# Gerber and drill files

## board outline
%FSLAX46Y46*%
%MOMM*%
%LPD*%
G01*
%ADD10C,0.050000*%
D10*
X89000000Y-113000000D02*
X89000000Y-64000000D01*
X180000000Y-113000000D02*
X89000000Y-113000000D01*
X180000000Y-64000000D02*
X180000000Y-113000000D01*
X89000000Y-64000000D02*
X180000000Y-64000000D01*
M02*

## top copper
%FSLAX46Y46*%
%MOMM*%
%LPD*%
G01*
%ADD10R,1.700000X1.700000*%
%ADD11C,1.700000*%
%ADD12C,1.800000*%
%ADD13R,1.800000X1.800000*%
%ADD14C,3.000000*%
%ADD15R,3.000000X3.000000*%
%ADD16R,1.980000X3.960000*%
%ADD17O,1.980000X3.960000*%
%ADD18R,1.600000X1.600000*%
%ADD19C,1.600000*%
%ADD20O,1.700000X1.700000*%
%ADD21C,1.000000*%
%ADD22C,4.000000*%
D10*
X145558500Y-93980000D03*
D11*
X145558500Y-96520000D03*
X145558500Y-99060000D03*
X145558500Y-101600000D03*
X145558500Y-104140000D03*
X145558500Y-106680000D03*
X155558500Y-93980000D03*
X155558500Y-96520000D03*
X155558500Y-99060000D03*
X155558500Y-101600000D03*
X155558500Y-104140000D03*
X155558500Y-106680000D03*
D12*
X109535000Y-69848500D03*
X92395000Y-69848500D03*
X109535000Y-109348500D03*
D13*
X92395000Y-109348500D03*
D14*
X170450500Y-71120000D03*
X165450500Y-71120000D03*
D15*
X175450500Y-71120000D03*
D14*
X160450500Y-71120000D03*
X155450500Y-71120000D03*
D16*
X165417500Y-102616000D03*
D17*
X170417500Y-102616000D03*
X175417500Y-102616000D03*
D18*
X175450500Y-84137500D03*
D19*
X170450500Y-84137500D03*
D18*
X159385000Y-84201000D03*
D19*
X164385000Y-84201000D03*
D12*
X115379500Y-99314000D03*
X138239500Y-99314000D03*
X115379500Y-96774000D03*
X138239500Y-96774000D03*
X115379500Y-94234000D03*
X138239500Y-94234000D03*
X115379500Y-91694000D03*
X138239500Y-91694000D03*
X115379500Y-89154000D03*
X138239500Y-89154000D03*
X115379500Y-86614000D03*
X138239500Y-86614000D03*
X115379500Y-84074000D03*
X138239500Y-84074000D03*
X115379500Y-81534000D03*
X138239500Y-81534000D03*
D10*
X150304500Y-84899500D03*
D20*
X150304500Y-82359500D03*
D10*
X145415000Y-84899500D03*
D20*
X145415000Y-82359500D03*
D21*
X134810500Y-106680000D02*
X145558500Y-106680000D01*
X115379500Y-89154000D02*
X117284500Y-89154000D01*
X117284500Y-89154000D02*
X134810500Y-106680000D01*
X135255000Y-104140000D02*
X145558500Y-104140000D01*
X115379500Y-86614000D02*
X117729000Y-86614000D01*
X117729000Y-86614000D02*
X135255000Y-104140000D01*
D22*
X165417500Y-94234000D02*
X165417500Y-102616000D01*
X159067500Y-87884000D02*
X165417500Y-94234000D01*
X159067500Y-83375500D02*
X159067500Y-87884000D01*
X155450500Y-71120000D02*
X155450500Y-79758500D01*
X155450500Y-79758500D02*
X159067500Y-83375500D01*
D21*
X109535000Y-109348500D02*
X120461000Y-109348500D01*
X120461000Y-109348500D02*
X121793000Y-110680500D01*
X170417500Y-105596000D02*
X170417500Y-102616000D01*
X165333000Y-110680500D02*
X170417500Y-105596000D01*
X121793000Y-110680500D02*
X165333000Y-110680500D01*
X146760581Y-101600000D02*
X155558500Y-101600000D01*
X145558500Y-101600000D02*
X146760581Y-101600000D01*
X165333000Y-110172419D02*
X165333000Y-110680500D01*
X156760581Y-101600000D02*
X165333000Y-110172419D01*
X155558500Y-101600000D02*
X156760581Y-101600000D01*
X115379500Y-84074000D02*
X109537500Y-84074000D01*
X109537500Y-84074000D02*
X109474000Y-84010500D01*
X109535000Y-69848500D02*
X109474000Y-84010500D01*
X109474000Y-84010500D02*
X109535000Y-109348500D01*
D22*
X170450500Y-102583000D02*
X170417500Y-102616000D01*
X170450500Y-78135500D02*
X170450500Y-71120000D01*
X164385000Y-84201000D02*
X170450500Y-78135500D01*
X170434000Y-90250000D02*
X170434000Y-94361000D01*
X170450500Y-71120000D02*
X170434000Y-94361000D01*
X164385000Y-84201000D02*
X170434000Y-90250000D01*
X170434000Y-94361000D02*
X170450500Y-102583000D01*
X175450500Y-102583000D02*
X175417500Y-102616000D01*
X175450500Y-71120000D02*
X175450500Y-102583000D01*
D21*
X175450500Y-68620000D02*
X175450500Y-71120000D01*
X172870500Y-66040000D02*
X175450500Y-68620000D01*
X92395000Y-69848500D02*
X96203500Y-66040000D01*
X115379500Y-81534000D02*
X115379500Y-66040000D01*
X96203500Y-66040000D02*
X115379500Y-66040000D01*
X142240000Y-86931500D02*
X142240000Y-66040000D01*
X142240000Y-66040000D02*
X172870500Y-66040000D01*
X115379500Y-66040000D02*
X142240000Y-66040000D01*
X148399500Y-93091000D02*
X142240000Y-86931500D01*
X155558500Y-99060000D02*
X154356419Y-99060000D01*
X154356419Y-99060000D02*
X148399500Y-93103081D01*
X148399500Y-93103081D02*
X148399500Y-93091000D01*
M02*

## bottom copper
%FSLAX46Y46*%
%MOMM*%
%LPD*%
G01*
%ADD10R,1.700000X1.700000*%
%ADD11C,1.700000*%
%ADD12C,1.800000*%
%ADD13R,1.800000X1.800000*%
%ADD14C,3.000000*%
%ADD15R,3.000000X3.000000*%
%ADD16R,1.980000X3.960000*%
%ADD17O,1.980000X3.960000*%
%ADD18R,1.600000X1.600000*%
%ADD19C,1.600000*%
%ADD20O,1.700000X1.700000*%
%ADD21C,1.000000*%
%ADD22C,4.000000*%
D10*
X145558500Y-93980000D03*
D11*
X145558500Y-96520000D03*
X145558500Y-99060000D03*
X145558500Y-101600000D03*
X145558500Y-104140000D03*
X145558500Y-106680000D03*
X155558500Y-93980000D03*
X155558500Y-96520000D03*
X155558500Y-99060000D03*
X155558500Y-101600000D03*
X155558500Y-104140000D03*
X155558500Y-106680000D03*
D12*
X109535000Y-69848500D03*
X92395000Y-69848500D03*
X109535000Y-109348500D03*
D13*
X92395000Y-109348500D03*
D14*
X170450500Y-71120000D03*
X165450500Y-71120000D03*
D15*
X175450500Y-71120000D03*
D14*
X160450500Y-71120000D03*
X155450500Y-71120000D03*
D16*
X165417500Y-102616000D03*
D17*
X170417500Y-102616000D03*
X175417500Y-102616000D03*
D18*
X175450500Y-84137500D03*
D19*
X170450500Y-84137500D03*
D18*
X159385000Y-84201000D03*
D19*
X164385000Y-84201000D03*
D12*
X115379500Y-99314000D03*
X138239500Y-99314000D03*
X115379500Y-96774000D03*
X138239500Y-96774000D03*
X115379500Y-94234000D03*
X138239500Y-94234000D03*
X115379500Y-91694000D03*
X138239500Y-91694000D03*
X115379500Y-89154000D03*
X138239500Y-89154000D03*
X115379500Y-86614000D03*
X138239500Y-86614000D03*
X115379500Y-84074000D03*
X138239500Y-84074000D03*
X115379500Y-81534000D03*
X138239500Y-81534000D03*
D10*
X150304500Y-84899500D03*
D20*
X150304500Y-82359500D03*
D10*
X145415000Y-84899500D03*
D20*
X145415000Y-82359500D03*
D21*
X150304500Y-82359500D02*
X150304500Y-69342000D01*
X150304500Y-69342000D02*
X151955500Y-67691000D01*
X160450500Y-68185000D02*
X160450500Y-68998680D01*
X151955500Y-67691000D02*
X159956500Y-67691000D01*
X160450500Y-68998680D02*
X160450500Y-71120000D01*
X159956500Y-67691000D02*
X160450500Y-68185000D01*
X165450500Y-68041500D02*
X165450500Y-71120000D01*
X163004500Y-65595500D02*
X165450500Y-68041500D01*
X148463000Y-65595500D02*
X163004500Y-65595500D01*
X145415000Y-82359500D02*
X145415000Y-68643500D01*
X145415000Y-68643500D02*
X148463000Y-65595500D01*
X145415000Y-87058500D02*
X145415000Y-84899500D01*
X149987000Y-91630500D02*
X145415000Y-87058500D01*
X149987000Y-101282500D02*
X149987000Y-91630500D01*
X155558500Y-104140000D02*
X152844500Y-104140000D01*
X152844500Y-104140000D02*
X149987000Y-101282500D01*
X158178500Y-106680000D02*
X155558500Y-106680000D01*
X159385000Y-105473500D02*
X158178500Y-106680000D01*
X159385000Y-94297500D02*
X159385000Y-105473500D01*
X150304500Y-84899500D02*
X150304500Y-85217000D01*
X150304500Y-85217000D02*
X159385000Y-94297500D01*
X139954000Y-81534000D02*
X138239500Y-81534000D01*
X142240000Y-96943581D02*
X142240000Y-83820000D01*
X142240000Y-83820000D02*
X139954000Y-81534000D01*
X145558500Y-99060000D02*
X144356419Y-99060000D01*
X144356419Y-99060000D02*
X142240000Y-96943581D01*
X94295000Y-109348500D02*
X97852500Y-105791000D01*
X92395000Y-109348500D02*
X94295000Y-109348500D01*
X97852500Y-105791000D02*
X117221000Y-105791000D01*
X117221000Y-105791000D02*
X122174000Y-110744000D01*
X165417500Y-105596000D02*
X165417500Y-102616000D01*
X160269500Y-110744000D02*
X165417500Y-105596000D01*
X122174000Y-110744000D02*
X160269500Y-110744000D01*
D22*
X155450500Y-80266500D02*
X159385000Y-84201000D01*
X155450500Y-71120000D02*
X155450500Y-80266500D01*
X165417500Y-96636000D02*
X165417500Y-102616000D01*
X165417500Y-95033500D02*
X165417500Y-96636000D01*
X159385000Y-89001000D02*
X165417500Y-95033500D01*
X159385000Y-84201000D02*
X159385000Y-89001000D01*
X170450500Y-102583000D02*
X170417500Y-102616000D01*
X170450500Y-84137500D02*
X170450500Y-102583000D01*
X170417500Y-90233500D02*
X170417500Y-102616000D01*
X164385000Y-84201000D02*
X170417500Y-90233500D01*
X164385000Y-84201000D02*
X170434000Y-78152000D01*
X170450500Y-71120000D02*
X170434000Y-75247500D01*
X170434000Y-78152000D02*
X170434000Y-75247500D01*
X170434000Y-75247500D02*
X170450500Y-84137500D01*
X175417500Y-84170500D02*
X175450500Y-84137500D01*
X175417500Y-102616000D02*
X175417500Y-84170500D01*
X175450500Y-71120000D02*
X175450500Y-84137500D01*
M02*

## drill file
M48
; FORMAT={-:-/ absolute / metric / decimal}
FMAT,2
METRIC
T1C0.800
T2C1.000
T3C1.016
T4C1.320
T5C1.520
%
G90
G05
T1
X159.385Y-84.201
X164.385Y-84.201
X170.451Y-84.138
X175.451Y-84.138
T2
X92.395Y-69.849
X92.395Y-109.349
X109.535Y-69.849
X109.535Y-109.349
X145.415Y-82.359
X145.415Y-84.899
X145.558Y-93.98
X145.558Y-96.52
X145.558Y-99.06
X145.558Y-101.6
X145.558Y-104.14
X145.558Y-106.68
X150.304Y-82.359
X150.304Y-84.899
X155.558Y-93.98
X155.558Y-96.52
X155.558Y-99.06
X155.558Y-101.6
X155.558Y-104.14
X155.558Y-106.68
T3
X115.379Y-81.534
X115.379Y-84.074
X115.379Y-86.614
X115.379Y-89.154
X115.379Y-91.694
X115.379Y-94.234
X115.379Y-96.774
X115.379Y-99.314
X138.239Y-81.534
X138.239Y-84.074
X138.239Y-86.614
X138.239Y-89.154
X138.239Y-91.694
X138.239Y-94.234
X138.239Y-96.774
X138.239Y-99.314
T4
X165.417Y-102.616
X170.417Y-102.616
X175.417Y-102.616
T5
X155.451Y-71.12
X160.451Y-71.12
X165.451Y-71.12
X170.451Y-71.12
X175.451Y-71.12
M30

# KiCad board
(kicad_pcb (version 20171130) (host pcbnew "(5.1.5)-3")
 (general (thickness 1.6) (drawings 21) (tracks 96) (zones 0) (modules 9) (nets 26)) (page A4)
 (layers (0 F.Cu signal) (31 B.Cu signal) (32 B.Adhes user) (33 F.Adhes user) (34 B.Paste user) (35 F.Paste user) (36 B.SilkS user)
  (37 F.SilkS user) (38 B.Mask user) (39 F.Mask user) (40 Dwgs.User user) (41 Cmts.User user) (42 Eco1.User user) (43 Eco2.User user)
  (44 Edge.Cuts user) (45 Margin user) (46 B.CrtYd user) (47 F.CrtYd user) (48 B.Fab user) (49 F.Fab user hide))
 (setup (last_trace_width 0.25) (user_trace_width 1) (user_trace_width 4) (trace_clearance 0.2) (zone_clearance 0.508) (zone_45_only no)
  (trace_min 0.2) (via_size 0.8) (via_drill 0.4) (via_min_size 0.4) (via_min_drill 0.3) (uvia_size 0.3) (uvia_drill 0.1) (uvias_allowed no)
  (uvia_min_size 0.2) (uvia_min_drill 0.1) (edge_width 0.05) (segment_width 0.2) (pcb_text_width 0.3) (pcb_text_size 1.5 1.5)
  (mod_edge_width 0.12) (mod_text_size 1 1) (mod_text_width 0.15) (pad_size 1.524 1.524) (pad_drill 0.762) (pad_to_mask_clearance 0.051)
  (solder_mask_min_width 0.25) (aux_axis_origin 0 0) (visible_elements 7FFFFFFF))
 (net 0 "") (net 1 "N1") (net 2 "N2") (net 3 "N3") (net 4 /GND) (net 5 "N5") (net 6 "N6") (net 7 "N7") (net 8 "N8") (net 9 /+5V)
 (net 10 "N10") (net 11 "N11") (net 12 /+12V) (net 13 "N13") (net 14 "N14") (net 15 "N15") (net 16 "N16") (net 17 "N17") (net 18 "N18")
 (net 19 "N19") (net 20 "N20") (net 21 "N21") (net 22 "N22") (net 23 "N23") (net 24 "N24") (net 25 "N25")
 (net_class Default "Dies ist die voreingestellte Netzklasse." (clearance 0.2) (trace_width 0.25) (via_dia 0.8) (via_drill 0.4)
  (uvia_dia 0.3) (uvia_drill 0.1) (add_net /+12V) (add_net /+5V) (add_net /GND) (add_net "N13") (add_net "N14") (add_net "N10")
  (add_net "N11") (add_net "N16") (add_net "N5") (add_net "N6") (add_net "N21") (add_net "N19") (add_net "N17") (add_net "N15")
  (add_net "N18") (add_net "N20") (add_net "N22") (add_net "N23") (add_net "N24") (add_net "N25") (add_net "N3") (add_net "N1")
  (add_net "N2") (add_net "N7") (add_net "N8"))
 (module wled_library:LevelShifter (layer F.Cu) (at 150.5585 100.33)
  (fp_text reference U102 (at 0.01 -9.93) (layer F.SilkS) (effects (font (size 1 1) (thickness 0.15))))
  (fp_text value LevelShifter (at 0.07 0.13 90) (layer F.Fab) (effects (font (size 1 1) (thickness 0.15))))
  (pad 1 thru_hole rect (at -5 -6.35) (size 1.7 1.7) (drill 1) (layers *.Cu *.Mask) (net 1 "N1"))
  (pad 2 thru_hole circle (at -5 -3.81) (size 1.7 1.7) (drill 1) (layers *.Cu *.Mask) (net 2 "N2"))
  (pad 3 thru_hole circle (at -5 -1.27) (size 1.7 1.7) (drill 1) (layers *.Cu *.Mask) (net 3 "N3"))
  (pad 4 thru_hole circle (at -5 1.27) (size 1.7 1.7) (drill 1) (layers *.Cu *.Mask) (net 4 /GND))
  (pad 5 thru_hole circle (at -5 3.81) (size 1.7 1.7) (drill 1) (layers *.Cu *.Mask) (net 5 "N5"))
  (pad 6 thru_hole circle (at -5 6.35) (size 1.7 1.7) (drill 1) (layers *.Cu *.Mask) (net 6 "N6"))
  (pad 7 thru_hole circle (at 5 -6.35) (size 1.7 1.7) (drill 1) (layers *.Cu *.Mask) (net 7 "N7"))
  (pad 8 thru_hole circle (at 5 -3.81) (size 1.7 1.7) (drill 1) (layers *.Cu *.Mask) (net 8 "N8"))
  (pad 9 thru_hole circle (at 5 -1.27) (size 1.7 1.7) (drill 1) (layers *.Cu *.Mask) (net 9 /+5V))
  (pad 10 thru_hole circle (at 5 1.27) (size 1.7 1.7) (drill 1) (layers *.Cu *.Mask) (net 4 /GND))
  (pad 11 thru_hole circle (at 5 3.81) (size 1.7 1.7) (drill 1) (layers *.Cu *.Mask) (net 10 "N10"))
  (pad 12 thru_hole circle (at 5 6.35) (size 1.7 1.7) (drill 1) (layers *.Cu *.Mask) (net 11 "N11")))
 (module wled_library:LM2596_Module (layer F.Cu) (at 100.965 89.5985 90)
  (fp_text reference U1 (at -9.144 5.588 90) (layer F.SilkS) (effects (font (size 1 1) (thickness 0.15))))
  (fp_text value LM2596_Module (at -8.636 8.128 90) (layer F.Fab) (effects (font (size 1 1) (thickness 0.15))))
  (pad 4 thru_hole circle (at 19.75 8.57 90) (size 1.8 1.8) (drill 1) (layers *.Cu *.Mask) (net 4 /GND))
  (pad 3 thru_hole circle (at 19.75 -8.57 90) (size 1.8 1.8) (drill 1) (layers *.Cu *.Mask) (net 9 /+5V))
  (pad 2 thru_hole circle (at -19.75 8.57 90) (size 1.8 1.8) (drill 1) (layers *.Cu *.Mask) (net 4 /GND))
  (pad 1 thru_hole rect (at -19.75 -8.57 90) (size 1.8 1.8) (drill 1) (layers *.Cu *.Mask) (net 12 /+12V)))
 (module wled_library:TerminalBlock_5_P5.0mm (layer F.Cu) (at 175.4505 71.12 180)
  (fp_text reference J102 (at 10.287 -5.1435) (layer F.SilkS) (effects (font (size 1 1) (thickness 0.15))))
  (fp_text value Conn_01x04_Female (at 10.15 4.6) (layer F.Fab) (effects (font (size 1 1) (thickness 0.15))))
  (pad 2 thru_hole circle (at 5 0 180) (size 3 3) (drill 1.52) (layers *.Cu *.Mask) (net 4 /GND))
  (pad 3 thru_hole circle (at 10 0 180) (size 3 3) (drill 1.52) (layers *.Cu *.Mask) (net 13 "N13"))
  (pad 1 thru_hole rect (at 0 0 180) (size 3 3) (drill 1.52) (layers *.Cu *.Mask) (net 9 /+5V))
  (pad 4 thru_hole circle (at 15 0 180) (size 3 3) (drill 1.52) (layers *.Cu *.Mask) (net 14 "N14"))
  (pad 5 thru_hole circle (at 20 0 180) (size 3 3) (drill 1.52) (layers *.Cu *.Mask) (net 12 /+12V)))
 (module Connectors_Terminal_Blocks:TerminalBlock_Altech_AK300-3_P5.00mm (layer F.Cu) (at 165.4175 102.616)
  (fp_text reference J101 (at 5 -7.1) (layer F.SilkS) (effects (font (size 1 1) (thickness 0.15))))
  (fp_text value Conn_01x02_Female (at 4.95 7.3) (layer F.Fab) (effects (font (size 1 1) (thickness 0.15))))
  (pad 1 thru_hole rect (at 0 0) (size 1.98 3.96) (drill 1.32) (layers *.Cu *.Mask) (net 12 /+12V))
  (pad 2 thru_hole oval (at 5 0) (size 1.98 3.96) (drill 1.32) (layers *.Cu *.Mask) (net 4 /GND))
  (pad 3 thru_hole oval (at 10 0) (size 1.98 3.96) (drill 1.32) (layers *.Cu *.Mask) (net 9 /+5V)))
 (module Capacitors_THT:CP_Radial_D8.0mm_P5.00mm (layer F.Cu) (at 175.4505 84.1375 180)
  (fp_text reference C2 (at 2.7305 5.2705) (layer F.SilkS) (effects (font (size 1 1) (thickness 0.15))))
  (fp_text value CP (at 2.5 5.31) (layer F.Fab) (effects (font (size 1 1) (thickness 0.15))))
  (pad 1 thru_hole rect (at 0 0 180) (size 1.6 1.6) (drill 0.8) (layers *.Cu *.Mask) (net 9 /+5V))
  (pad 2 thru_hole circle (at 5 0 180) (size 1.6 1.6) (drill 0.8) (layers *.Cu *.Mask) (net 4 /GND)))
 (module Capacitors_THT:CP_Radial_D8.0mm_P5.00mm (layer F.Cu) (at 159.385 84.201)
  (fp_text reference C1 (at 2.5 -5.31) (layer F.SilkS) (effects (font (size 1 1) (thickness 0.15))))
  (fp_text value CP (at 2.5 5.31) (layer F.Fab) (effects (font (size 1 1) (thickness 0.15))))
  (pad 1 thru_hole rect (at 0 0) (size 1.6 1.6) (drill 0.8) (layers *.Cu *.Mask) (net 12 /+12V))
  (pad 2 thru_hole circle (at 5 0) (size 1.6 1.6) (drill 0.8) (layers *.Cu *.Mask) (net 4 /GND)))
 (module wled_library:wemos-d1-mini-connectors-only (layer F.Cu) (at 126.8095 90.424 270)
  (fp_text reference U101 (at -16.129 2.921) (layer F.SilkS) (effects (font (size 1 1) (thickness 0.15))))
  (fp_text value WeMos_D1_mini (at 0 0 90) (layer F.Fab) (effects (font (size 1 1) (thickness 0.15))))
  (pad 16 thru_hole circle (at 8.89 11.43 270) (size 1.8 1.8) (drill 1.016) (layers *.Cu *.Mask) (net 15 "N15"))
  (pad 1 thru_hole circle (at 8.89 -11.43 270) (size 1.8 1.8) (drill 1.016) (layers *.Cu *.Mask) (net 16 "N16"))
  (pad 15 thru_hole circle (at 6.35 11.43 270) (size 1.8 1.8) (drill 1.016) (layers *.Cu *.Mask) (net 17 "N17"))
  (pad 2 thru_hole circle (at 6.35 -11.43 270) (size 1.8 1.8) (drill 1.016) (layers *.Cu *.Mask) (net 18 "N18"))
  (pad 14 thru_hole circle (at 3.81 11.43 270) (size 1.8 1.8) (drill 1.016) (layers *.Cu *.Mask) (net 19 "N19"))
  (pad 3 thru_hole circle (at 3.81 -11.43 270) (size 1.8 1.8) (drill 1.016) (layers *.Cu *.Mask) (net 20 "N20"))
  (pad 13 thru_hole circle (at 1.27 11.43 270) (size 1.8 1.8) (drill 1.016) (layers *.Cu *.Mask) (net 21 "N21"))
  (pad 4 thru_hole circle (at 1.27 -11.43 270) (size 1.8 1.8) (drill 1.016) (layers *.Cu *.Mask) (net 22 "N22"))
  (pad 12 thru_hole circle (at -1.27 11.43 270) (size 1.8 1.8) (drill 1.016) (layers *.Cu *.Mask) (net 6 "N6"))
  (pad 5 thru_hole circle (at -1.27 -11.43 270) (size 1.8 1.8) (drill 1.016) (layers *.Cu *.Mask) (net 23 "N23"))
  (pad 11 thru_hole circle (at -3.81 11.43 270) (size 1.8 1.8) (drill 1.016) (layers *.Cu *.Mask) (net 5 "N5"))
  (pad 6 thru_hole circle (at -3.81 -11.43 270) (size 1.8 1.8) (drill 1.016) (layers *.Cu *.Mask) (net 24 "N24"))
  (pad 10 thru_hole circle (at -6.35 11.43 270) (size 1.8 1.8) (drill 1.016) (layers *.Cu *.Mask) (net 4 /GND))
  (pad 7 thru_hole circle (at -6.35 -11.43 270) (size 1.8 1.8) (drill 1.016) (layers *.Cu *.Mask) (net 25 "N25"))
  (pad 9 thru_hole circle (at -8.89 11.43 270) (size 1.8 1.8) (drill 1.016) (layers *.Cu *.Mask) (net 9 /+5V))
  (pad 8 thru_hole circle (at -8.89 -11.43 270) (size 1.8 1.8) (drill 1.016) (layers *.Cu *.Mask) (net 3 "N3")))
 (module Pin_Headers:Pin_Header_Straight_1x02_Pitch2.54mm (layer F.Cu) (at 150.3045 84.8995 180)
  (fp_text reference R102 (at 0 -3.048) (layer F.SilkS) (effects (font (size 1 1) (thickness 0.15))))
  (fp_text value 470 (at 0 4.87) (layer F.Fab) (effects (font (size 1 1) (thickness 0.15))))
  (pad 1 thru_hole rect (at 0 0 180) (size 1.7 1.7) (drill 1) (layers *.Cu *.Mask) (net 11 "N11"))
  (pad 2 thru_hole oval (at 0 2.54 180) (size 1.7 1.7) (drill 1) (layers *.Cu *.Mask) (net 14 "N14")))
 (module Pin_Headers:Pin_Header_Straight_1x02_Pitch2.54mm (layer F.Cu) (at 145.415 84.8995 180)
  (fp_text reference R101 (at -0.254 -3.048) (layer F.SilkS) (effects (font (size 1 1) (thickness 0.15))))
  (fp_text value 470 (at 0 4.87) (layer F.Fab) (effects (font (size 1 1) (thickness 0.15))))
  (pad 1 thru_hole rect (at 0 0 180) (size 1.7 1.7) (drill 1) (layers *.Cu *.Mask) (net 10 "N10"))
  (pad 2 thru_hole oval (at 0 2.54 180) (size 1.7 1.7) (drill 1) (layers *.Cu *.Mask) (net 13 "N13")))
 (gr_line (start 89 113) (end 89 64) (layer Edge.Cuts) (width 0.05))
 (gr_line (start 180 113) (end 89 113) (layer Edge.Cuts) (width 0.05))
 (gr_line (start 180 64) (end 180 113) (layer Edge.Cuts) (width 0.05))
 (gr_line (start 89 64) (end 180 64) (layer Edge.Cuts) (width 0.05))
 (segment (start 150.3045 82.3595) (end 150.3045 69.342) (width 1) (layer B.Cu) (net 14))
 (segment (start 150.3045 69.342) (end 151.9555 67.691) (width 1) (layer B.Cu) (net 14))
 (segment (start 160.4505 68.185) (end 160.4505 68.99868) (width 1) (layer B.Cu) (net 14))
 (segment (start 151.9555 67.691) (end 159.9565 67.691) (width 1) (layer B.Cu) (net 14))
 (segment (start 160.4505 68.99868) (end 160.4505 71.12) (width 1) (layer B.Cu) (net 14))
 (segment (start 159.9565 67.691) (end 160.4505 68.185) (width 1) (layer B.Cu) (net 14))
 (segment (start 165.4505 68.0415) (end 165.4505 71.12) (width 1) (layer B.Cu) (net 13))
 (segment (start 163.0045 65.5955) (end 165.4505 68.0415) (width 1) (layer B.Cu) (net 13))
 (segment (start 148.463 65.5955) (end 163.0045 65.5955) (width 1) (layer B.Cu) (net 13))
 (segment (start 145.415 82.3595) (end 145.415 68.6435) (width 1) (layer B.Cu) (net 13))
 (segment (start 145.415 68.6435) (end 148.463 65.5955) (width 1) (layer B.Cu) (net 13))
 (segment (start 145.415 87.0585) (end 145.415 84.8995) (width 1) (layer B.Cu) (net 10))
 (segment (start 149.987 91.6305) (end 145.415 87.0585) (width 1) (layer B.Cu) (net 10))
 (segment (start 149.987 101.2825) (end 149.987 91.6305) (width 1) (layer B.Cu) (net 10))
 (segment (start 155.5585 104.14) (end 152.8445 104.14) (width 1) (layer B.Cu) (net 10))
 (segment (start 152.8445 104.14) (end 149.987 101.2825) (width 1) (layer B.Cu) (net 10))
 (segment (start 158.1785 106.68) (end 155.5585 106.68) (width 1) (layer B.Cu) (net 11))
 (segment (start 159.385 105.4735) (end 158.1785 106.68) (width 1) (layer B.Cu) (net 11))
 (segment (start 159.385 94.2975) (end 159.385 105.4735) (width 1) (layer B.Cu) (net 11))
 (segment (start 150.3045 84.8995) (end 150.3045 85.217) (width 1) (layer B.Cu) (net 11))
 (segment (start 150.3045 85.217) (end 159.385 94.2975) (width 1) (layer B.Cu) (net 11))
 (segment (start 134.8105 106.68) (end 145.5585 106.68) (width 1) (layer F.Cu) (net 6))
 (segment (start 115.3795 89.154) (end 117.2845 89.154) (width 1) (layer F.Cu) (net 6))
 (segment (start 117.2845 89.154) (end 134.8105 106.68) (width 1) (layer F.Cu) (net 6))
 (segment (start 135.255 104.14) (end 145.5585 104.14) (width 1) (layer F.Cu) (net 5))
 (segment (start 115.3795 86.614) (end 117.729 86.614) (width 1) (layer F.Cu) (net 5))
 (segment (start 117.729 86.614) (end 135.255 104.14) (width 1) (layer F.Cu) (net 5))
 (segment (start 139.954 81.534) (end 138.2395 81.534) (width 1) (layer B.Cu) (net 3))
 (segment (start 142.24 96.943581) (end 142.24 83.82) (width 1) (layer B.Cu) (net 3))
 (segment (start 142.24 83.82) (end 139.954 81.534) (width 1) (layer B.Cu) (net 3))
 (segment (start 145.5585 99.06) (end 144.356419 99.06) (width 1) (layer B.Cu) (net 3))
 (segment (start 144.356419 99.06) (end 142.24 96.943581) (width 1) (layer B.Cu) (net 3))
 (segment (start 94.295 109.3485) (end 97.8525 105.791) (width 1) (layer B.Cu) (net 12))
 (segment (start 92.395 109.3485) (end 94.295 109.3485) (width 1) (layer B.Cu) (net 12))
 (segment (start 97.8525 105.791) (end 117.221 105.791) (width 1) (layer B.Cu) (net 12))
 (segment (start 117.221 105.791) (end 122.174 110.744) (width 1) (layer B.Cu) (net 12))
 (segment (start 165.4175 105.596) (end 165.4175 102.616) (width 1) (layer B.Cu) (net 12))
 (segment (start 160.2695 110.744) (end 165.4175 105.596) (width 1) (layer B.Cu) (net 12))
 (segment (start 122.174 110.744) (end 160.2695 110.744) (width 1) (layer B.Cu) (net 12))
 (segment (start 155.4505 80.2665) (end 159.385 84.201) (width 4) (layer B.Cu) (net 12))
 (segment (start 155.4505 71.12) (end 155.4505 80.2665) (width 4) (layer B.Cu) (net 12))
 (segment (start 165.4175 96.636) (end 165.4175 102.616) (width 4) (layer B.Cu) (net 12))
 (segment (start 165.4175 95.0335) (end 165.4175 96.636) (width 4) (layer B.Cu) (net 12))
 (segment (start 159.385 89.001) (end 165.4175 95.0335) (width 4) (layer B.Cu) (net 12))
 (segment (start 159.385 84.201) (end 159.385 89.001) (width 4) (layer B.Cu) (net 12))
 (segment (start 165.4175 94.234) (end 165.4175 102.616) (width 4) (layer F.Cu) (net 12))
 (segment (start 159.0675 87.884) (end 165.4175 94.234) (width 4) (layer F.Cu) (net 12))
 (segment (start 159.0675 83.3755) (end 159.0675 87.884) (width 4) (layer F.Cu) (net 12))
 (segment (start 155.4505 71.12) (end 155.4505 79.7585) (width 4) (layer F.Cu) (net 12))
 (segment (start 155.4505 79.7585) (end 159.0675 83.3755) (width 4) (layer F.Cu) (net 12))
 (segment (start 170.4505 102.583) (end 170.4175 102.616) (width 4) (layer B.Cu) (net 4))
 (segment (start 170.4505 84.1375) (end 170.4505 102.583) (width 4) (layer B.Cu) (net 4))
 (segment (start 170.4175 90.2335) (end 170.4175 102.616) (width 4) (layer B.Cu) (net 4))
 (segment (start 164.385 84.201) (end 170.4175 90.2335) (width 4) (layer B.Cu) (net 4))
 (segment (start 109.535 109.3485) (end 120.461 109.3485) (width 1) (layer F.Cu) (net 4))
 (segment (start 120.461 109.3485) (end 121.793 110.6805) (width 1) (layer F.Cu) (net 4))
 (segment (start 170.4175 105.596) (end 170.4175 102.616) (width 1) (layer F.Cu) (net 4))
 (segment (start 165.333 110.6805) (end 170.4175 105.596) (width 1) (layer F.Cu) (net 4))
 (segment (start 121.793 110.6805) (end 165.333 110.6805) (width 1) (layer F.Cu) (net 4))
 (segment (start 146.760581 101.6) (end 155.5585 101.6) (width 1) (layer F.Cu) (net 4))
 (segment (start 145.5585 101.6) (end 146.760581 101.6) (width 1) (layer F.Cu) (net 4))
 (segment (start 165.333 110.172419) (end 165.333 110.6805) (width 1) (layer F.Cu) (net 4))
 (segment (start 156.760581 101.6) (end 165.333 110.172419) (width 1) (layer F.Cu) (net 4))
 (segment (start 155.5585 101.6) (end 156.760581 101.6) (width 1) (layer F.Cu) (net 4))
 (segment (start 115.3795 84.074) (end 109.5375 84.074) (width 1) (layer F.Cu) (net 4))
 (segment (start 109.5375 84.074) (end 109.474 84.0105) (width 1) (layer F.Cu) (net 4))
 (segment (start 109.535 69.8485) (end 109.474 84.0105) (width 1) (layer F.Cu) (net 4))
 (segment (start 109.474 84.0105) (end 109.535 109.3485) (width 1) (layer F.Cu) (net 4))
 (segment (start 170.4505 102.583) (end 170.4175 102.616) (width 4) (layer F.Cu) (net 4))
 (segment (start 170.4505 78.1355) (end 170.4505 71.12) (width 4) (layer F.Cu) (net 4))
 (segment (start 164.385 84.201) (end 170.4505 78.1355) (width 4) (layer F.Cu) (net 4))
 (segment (start 170.434 90.25) (end 170.434 94.361) (width 4) (layer F.Cu) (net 4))
 (segment (start 170.4505 71.12) (end 170.434 94.361) (width 4) (layer F.Cu) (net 4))
 (segment (start 164.385 84.201) (end 170.434 90.25) (width 4) (layer F.Cu) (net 4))
 (segment (start 170.434 94.361) (end 170.4505 102.583) (width 4) (layer F.Cu) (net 4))
 (segment (start 164.385 84.201) (end 170.434 78.152) (width 4) (layer B.Cu) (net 4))
 (segment (start 170.4505 71.12) (end 170.434 75.2475) (width 4) (layer B.Cu) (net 4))
 (segment (start 170.434 78.152) (end 170.434 75.2475) (width 4) (layer B.Cu) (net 4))
 (segment (start 170.434 75.2475) (end 170.4505 84.1375) (width 4) (layer B.Cu) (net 4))
 (segment (start 175.4175 84.1705) (end 175.4505 84.1375) (width 4) (layer B.Cu) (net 9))
 (segment (start 175.4175 102.616) (end 175.4175 84.1705) (width 4) (layer B.Cu) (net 9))
 (segment (start 175.4505 71.12) (end 175.4505 84.1375) (width 4) (layer B.Cu) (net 9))
 (segment (start 175.4505 102.583) (end 175.4175 102.616) (width 4) (layer F.Cu) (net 9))
 (segment (start 175.4505 71.12) (end 175.4505 102.583) (width 4) (layer F.Cu) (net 9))
 (segment (start 175.4505 68.62) (end 175.4505 71.12) (width 1) (layer F.Cu) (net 9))
 (segment (start 172.8705 66.04) (end 175.4505 68.62) (width 1) (layer F.Cu) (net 9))
 (segment (start 92.395 69.8485) (end 96.2035 66.04) (width 1) (layer F.Cu) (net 9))
 (segment (start 115.3795 81.534) (end 115.3795 66.04) (width 1) (layer F.Cu) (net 9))
 (segment (start 96.2035 66.04) (end 115.3795 66.04) (width 1) (layer F.Cu) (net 9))
 (segment (start 142.24 86.9315) (end 142.24 66.04) (width 1) (layer F.Cu) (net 9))
 (segment (start 142.24 66.04) (end 172.8705 66.04) (width 1) (layer F.Cu) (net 9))
 (segment (start 115.3795 66.04) (end 142.24 66.04) (width 1) (layer F.Cu) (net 9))
 (segment (start 148.3995 93.091) (end 142.24 86.9315) (width 1) (layer F.Cu) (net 9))
 (segment (start 155.5585 99.06) (end 154.356419 99.06) (width 1) (layer F.Cu) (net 9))
 (segment (start 154.356419 99.06) (end 148.3995 93.103081) (width 1) (layer F.Cu) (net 9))
 (segment (start 148.3995 93.103081) (end 148.3995 93.091) (width 1) (layer F.Cu) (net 9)))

